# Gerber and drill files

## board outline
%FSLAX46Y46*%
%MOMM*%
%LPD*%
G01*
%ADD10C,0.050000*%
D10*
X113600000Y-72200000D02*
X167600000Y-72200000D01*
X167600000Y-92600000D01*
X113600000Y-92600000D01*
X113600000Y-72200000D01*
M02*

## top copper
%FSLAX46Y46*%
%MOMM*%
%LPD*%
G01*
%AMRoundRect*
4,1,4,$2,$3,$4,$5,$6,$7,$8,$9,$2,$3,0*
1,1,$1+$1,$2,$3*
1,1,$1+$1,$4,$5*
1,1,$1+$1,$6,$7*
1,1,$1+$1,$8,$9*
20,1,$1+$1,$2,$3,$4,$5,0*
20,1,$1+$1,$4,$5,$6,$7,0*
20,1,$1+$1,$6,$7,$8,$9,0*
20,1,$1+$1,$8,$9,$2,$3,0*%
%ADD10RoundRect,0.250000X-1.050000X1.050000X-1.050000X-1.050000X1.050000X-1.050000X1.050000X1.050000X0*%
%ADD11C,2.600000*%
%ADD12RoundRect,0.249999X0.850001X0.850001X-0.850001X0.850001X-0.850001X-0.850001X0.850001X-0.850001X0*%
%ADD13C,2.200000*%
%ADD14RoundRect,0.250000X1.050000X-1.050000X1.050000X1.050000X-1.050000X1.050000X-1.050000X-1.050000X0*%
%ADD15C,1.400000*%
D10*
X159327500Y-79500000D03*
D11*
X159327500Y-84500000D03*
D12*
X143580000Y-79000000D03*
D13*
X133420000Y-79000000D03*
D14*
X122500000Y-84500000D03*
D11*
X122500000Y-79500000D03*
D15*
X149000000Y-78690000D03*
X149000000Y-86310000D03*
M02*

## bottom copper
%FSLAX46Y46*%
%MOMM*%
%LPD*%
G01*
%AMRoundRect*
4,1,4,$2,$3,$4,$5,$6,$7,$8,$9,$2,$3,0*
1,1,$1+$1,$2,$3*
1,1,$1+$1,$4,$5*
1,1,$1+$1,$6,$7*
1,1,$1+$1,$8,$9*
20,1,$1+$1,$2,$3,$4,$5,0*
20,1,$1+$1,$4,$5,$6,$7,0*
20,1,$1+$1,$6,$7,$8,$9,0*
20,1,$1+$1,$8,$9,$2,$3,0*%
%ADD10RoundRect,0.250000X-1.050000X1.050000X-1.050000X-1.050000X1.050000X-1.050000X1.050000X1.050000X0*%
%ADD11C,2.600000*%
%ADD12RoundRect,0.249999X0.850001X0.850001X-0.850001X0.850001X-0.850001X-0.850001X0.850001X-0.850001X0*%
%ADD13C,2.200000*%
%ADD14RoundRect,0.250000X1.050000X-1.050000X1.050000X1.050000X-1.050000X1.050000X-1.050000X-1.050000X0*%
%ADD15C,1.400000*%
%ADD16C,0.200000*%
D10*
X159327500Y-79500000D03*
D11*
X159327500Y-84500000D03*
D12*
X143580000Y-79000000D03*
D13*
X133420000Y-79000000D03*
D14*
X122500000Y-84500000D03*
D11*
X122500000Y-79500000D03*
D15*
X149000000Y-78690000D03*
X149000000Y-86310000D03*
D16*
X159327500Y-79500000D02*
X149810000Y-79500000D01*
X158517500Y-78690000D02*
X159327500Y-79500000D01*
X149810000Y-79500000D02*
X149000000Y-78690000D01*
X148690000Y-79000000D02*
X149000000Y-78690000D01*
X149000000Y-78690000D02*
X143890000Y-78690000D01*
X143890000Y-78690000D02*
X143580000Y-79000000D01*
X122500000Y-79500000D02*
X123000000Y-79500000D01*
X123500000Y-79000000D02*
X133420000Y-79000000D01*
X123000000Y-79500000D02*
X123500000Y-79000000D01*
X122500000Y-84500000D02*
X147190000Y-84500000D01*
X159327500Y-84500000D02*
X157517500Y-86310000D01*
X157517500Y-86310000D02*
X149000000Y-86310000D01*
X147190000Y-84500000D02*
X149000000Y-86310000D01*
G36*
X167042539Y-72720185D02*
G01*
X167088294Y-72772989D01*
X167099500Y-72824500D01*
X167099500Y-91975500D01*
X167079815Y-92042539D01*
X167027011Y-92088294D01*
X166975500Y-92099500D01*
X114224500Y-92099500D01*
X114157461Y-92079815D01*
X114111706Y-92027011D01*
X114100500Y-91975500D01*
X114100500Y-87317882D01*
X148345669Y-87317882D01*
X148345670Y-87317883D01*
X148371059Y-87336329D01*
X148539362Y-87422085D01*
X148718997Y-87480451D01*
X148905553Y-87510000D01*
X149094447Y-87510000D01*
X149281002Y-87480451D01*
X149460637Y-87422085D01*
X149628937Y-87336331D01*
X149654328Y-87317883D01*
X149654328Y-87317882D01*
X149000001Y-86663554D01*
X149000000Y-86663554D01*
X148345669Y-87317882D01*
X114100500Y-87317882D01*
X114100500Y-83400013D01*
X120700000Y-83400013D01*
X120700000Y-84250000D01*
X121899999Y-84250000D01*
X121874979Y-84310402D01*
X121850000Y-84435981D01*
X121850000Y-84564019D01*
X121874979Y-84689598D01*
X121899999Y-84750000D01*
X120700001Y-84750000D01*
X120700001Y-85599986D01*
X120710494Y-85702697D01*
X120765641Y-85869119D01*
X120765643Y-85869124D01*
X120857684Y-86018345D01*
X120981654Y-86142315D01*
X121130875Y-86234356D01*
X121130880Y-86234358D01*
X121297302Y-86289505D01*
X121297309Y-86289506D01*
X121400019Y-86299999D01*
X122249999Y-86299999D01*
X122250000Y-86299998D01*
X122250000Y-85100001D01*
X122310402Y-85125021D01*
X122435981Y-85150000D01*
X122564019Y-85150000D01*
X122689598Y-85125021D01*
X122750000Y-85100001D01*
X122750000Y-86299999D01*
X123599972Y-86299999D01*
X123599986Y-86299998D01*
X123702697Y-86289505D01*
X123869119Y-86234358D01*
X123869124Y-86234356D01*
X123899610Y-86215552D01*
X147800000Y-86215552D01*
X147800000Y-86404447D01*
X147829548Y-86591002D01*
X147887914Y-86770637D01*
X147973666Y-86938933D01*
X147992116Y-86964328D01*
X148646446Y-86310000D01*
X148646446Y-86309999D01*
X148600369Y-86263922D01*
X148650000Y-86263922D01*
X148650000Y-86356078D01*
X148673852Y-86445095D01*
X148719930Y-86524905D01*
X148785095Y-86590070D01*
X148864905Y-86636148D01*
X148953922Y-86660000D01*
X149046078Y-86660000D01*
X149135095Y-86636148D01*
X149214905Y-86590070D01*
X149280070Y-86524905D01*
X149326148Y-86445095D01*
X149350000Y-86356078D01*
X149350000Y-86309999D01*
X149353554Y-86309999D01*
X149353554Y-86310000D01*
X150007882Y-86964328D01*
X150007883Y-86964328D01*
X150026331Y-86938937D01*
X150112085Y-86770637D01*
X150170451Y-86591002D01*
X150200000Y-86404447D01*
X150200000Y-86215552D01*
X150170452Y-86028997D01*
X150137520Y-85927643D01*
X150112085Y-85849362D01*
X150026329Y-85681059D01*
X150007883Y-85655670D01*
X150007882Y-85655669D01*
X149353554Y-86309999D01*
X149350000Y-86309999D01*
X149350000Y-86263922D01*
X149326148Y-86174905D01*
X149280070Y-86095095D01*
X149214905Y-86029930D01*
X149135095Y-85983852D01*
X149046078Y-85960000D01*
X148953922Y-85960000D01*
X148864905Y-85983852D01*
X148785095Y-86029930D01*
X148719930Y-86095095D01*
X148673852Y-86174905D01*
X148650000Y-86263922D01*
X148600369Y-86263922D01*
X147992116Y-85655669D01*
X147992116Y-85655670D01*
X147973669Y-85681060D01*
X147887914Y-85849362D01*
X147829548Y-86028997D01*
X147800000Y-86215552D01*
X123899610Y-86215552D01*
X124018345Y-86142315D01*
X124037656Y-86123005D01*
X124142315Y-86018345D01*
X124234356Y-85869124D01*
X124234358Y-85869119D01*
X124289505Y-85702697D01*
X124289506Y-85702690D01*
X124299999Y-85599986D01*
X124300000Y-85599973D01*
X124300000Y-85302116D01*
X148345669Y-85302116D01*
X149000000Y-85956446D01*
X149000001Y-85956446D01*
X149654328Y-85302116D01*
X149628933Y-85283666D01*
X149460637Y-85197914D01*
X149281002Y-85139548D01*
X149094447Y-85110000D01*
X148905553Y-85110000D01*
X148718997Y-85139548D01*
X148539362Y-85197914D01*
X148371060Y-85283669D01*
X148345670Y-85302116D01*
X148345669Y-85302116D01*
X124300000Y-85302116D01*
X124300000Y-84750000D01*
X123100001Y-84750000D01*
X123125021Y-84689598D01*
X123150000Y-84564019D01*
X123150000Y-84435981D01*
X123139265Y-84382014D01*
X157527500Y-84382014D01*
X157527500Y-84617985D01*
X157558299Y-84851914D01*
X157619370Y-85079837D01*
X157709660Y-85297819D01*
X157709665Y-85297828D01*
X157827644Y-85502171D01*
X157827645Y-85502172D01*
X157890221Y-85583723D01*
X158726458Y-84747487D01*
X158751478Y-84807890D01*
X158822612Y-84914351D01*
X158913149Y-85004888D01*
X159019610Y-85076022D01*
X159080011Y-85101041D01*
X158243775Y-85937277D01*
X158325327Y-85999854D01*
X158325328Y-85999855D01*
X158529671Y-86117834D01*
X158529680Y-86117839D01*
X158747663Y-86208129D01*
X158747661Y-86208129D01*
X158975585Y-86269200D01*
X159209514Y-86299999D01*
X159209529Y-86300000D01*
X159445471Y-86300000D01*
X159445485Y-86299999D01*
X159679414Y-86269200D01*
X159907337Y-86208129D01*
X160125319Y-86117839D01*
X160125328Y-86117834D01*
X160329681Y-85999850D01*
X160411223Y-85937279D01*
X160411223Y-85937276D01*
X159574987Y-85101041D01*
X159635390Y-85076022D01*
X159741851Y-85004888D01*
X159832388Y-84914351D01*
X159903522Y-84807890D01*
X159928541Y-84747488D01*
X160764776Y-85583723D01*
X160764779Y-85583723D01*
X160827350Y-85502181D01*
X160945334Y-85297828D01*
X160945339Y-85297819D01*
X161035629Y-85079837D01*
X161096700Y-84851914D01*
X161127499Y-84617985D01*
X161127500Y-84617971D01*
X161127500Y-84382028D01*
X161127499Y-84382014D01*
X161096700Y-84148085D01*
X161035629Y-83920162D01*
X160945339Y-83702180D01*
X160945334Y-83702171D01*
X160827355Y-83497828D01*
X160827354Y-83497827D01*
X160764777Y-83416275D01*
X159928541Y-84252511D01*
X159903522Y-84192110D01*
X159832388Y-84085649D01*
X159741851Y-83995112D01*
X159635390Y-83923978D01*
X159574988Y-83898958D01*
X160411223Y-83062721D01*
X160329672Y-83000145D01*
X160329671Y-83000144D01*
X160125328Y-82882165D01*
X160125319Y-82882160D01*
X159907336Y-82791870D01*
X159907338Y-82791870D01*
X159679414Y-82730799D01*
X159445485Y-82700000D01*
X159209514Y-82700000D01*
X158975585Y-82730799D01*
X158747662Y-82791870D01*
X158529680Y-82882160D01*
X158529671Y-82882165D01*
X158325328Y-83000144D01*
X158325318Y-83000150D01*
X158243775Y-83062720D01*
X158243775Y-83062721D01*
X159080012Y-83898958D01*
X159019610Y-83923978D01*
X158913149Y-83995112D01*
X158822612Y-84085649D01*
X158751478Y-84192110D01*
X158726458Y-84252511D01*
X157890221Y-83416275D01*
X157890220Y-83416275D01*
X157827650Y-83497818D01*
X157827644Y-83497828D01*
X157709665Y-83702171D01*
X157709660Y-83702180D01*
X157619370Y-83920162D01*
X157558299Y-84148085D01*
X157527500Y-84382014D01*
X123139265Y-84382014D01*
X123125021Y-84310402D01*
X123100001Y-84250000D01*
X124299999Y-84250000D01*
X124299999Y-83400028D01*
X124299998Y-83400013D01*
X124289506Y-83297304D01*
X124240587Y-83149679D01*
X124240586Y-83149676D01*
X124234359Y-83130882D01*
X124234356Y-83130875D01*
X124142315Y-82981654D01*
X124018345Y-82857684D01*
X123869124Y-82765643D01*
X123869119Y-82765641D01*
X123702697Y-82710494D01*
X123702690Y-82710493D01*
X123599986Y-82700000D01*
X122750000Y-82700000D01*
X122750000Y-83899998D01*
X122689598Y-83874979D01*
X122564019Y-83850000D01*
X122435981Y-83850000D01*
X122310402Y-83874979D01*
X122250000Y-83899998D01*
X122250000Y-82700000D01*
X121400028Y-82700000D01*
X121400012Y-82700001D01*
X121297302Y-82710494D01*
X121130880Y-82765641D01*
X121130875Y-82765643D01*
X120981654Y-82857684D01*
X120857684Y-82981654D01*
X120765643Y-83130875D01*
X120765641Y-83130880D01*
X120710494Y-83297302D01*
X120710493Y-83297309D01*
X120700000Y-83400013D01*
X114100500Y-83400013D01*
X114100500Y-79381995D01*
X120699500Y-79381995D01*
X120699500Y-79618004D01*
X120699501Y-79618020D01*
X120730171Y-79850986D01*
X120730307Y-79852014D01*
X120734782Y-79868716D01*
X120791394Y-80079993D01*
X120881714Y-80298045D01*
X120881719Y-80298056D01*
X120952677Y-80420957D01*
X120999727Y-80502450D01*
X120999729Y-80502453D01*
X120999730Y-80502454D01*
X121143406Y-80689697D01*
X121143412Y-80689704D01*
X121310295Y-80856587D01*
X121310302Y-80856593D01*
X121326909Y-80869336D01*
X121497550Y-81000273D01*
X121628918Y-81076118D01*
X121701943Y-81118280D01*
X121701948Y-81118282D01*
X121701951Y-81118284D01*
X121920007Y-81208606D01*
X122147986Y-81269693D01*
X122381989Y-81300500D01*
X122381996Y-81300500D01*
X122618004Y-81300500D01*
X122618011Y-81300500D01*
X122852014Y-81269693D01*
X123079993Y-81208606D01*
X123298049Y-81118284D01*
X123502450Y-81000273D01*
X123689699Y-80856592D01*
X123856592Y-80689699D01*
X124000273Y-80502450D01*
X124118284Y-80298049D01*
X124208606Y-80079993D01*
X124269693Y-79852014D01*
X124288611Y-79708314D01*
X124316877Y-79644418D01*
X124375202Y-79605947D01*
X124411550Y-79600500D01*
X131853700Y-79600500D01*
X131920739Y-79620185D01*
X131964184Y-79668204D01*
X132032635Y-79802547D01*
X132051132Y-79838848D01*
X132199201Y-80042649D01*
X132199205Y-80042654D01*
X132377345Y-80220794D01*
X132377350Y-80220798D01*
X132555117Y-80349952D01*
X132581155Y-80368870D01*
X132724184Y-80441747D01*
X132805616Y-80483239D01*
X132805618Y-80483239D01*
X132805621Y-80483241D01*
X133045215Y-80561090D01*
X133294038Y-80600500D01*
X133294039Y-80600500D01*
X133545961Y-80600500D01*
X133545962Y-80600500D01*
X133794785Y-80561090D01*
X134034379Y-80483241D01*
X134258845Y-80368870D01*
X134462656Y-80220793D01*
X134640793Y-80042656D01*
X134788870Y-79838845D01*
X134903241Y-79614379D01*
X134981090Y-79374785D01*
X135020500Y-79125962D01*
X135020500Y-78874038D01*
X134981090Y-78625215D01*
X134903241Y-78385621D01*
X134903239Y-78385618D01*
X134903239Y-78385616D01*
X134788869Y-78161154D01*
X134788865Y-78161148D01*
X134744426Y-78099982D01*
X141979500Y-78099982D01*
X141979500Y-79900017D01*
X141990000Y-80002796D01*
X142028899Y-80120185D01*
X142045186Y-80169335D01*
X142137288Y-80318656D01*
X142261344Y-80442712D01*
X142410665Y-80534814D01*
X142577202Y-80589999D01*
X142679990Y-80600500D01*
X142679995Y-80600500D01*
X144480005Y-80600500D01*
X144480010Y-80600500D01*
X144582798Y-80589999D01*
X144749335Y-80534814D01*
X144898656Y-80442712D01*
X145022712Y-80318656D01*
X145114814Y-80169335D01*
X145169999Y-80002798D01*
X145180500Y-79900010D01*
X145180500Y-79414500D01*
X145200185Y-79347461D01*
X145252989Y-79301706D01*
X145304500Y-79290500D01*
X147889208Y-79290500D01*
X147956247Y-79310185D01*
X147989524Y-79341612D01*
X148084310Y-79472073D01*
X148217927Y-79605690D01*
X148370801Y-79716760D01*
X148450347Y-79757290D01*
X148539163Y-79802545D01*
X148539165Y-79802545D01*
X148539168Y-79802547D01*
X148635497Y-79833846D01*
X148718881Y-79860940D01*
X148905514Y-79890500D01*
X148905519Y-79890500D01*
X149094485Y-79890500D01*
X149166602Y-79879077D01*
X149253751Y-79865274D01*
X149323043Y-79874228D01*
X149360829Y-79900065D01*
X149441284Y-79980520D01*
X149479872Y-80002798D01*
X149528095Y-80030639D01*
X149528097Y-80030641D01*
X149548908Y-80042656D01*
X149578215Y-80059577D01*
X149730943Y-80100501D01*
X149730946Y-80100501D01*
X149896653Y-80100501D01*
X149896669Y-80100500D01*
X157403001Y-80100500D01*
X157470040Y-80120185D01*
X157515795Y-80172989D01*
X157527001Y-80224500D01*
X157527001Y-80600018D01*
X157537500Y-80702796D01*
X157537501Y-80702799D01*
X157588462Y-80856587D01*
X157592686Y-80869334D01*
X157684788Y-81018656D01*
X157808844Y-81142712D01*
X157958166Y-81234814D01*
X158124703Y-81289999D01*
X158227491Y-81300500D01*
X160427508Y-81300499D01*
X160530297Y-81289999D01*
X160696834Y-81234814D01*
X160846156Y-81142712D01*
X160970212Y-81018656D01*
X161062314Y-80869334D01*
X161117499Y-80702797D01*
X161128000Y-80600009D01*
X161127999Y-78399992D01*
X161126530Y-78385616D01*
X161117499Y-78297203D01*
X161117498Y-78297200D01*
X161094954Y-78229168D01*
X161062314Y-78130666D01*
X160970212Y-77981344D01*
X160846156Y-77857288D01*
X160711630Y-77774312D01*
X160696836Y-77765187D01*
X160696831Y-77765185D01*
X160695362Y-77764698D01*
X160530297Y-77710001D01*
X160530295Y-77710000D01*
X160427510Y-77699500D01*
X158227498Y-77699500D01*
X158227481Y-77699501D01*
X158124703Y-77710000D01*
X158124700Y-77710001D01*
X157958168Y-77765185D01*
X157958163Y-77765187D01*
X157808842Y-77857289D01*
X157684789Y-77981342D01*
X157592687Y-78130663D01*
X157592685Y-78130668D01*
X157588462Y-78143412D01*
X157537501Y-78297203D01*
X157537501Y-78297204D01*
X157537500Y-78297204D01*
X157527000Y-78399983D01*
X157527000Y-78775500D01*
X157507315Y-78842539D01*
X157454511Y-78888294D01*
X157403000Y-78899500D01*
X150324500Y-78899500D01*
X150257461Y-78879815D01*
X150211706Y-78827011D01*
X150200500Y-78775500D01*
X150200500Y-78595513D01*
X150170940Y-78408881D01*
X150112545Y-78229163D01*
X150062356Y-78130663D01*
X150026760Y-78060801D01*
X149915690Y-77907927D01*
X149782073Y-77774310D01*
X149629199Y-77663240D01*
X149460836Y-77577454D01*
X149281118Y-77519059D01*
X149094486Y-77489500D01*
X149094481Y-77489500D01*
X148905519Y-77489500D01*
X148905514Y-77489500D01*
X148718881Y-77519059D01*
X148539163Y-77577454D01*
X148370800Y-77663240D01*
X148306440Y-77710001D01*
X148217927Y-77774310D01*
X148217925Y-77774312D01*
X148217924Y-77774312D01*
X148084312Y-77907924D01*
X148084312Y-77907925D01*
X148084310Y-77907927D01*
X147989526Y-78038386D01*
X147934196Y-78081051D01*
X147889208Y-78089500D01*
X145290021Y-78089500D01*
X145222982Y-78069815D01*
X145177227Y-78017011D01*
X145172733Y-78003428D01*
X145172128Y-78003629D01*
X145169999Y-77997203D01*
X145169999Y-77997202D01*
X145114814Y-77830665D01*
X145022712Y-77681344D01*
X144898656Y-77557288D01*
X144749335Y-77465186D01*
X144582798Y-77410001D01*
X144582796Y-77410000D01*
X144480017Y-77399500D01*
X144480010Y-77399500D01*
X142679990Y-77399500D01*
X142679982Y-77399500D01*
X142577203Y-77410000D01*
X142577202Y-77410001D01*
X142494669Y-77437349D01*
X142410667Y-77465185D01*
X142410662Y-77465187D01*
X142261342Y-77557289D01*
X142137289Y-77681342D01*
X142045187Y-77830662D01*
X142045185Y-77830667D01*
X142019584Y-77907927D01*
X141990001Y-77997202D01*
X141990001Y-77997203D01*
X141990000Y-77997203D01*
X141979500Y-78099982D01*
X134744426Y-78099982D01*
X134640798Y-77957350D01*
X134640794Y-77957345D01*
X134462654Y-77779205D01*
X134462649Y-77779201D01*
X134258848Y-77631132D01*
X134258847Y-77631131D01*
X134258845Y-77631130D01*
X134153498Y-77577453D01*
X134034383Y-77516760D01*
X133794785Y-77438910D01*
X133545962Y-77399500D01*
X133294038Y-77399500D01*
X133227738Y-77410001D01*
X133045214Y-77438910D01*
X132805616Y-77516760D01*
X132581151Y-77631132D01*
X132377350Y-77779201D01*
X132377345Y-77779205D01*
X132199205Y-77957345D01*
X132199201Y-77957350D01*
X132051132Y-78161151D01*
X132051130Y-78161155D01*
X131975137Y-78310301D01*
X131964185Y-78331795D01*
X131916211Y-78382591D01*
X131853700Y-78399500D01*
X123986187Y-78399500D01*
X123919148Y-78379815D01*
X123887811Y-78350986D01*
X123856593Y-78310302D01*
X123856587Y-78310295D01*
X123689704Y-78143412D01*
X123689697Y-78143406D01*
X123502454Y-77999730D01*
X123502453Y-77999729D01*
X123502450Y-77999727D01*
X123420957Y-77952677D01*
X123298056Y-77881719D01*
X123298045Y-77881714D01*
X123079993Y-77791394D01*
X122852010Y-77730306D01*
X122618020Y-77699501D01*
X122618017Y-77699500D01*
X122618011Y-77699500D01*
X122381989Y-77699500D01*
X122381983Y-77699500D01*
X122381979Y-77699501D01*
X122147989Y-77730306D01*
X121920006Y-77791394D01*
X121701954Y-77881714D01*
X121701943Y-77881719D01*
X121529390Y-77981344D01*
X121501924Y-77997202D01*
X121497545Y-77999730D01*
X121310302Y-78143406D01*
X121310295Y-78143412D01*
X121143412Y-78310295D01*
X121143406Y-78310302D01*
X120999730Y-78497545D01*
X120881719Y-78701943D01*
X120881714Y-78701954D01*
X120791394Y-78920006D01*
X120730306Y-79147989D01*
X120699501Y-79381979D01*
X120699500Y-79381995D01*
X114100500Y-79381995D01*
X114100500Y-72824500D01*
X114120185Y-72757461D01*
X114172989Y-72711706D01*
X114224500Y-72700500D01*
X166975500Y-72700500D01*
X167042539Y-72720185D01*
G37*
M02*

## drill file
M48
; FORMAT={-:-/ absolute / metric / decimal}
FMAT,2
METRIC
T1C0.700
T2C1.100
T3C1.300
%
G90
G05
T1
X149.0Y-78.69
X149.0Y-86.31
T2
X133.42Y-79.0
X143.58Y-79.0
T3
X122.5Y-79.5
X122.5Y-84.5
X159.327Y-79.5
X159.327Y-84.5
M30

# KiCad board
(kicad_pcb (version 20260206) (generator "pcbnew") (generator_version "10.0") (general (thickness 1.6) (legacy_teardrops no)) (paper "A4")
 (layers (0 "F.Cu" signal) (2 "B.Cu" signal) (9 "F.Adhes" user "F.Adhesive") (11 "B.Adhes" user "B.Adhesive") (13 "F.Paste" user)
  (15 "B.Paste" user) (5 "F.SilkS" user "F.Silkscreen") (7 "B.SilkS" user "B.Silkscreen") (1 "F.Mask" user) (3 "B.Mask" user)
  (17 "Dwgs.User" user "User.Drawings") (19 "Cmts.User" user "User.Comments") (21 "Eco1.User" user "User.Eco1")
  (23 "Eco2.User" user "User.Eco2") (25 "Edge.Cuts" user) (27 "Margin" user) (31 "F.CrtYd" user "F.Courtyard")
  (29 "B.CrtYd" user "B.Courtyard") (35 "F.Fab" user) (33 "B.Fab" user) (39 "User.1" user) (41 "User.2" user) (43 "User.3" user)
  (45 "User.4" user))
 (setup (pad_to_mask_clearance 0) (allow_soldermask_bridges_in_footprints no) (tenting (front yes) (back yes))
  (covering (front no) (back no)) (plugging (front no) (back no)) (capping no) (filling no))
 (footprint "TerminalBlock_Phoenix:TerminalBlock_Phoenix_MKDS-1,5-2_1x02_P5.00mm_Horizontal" (layer "F.Cu") (at 159.3275 79.5 -90)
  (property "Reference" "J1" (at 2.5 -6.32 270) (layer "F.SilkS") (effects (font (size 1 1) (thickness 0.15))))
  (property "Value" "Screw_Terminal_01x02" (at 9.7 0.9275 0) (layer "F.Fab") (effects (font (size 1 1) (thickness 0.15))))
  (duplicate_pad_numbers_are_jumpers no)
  (pad "1" thru_hole roundrect (at 0 0 270) (size 2.6 2.6) (drill 1.3) (layers "*.Cu" "*.Mask") (remove_unused_layers no)
   (roundrect_rratio 0.096154) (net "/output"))
  (pad "2" thru_hole circle (at 5 0 270) (size 2.6 2.6) (drill 1.3) (layers "*.Cu" "*.Mask") (remove_unused_layers no) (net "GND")))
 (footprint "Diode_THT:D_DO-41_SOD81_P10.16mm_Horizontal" (layer "F.Cu") (at 143.58 79 180)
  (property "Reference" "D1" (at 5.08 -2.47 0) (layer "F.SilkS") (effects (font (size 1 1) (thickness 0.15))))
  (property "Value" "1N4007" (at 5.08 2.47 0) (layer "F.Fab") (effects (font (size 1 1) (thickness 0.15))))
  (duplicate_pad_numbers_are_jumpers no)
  (pad "1" thru_hole roundrect (at 0 0 180) (size 2.2 2.2) (drill 1.1) (layers "*.Cu" "*.Mask") (remove_unused_layers no)
   (roundrect_rratio 0.113636) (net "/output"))
  (pad "2" thru_hole circle (at 10.16 0 180) (size 2.2 2.2) (drill 1.1) (layers "*.Cu" "*.Mask") (remove_unused_layers no) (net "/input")))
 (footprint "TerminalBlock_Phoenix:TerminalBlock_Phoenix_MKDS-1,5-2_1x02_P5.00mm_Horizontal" (layer "F.Cu") (at 122.5 84.5 90)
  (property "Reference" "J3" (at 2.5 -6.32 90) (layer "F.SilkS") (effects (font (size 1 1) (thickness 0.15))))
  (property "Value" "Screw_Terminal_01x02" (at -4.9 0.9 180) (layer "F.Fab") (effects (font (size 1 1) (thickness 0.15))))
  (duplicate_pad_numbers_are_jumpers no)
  (pad "1" thru_hole roundrect (at 0 0 90) (size 2.6 2.6) (drill 1.3) (layers "*.Cu" "*.Mask") (remove_unused_layers no)
   (roundrect_rratio 0.096154) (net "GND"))
  (pad "2" thru_hole circle (at 5 0 90) (size 2.6 2.6) (drill 1.3) (layers "*.Cu" "*.Mask") (remove_unused_layers no) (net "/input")))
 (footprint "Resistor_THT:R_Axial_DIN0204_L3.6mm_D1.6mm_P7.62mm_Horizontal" (layer "F.Cu") (at 149 78.69 -90)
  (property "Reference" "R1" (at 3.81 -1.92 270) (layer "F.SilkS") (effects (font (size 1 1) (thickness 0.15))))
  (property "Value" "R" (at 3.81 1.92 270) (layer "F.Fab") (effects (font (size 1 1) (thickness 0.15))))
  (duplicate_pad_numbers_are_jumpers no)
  (pad "1" thru_hole circle (at 0 0 270) (size 1.4 1.4) (drill 0.7) (layers "*.Cu" "*.Mask") (remove_unused_layers no) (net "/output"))
  (pad "2" thru_hole circle (at 7.62 0 270) (size 1.4 1.4) (drill 0.7) (layers "*.Cu" "*.Mask") (remove_unused_layers no) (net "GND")))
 (gr_rect (start 113.6 72.2) (end 167.6 92.6) (stroke (width 0.05) (type default)) (fill no) (layer "Edge.Cuts"))
 (segment (start 159.3275 79.5) (end 149.81 79.5) (width 0.2) (layer "B.Cu") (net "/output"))
 (segment (start 158.5175 78.69) (end 159.3275 79.5) (width 0.2) (layer "B.Cu") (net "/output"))
 (segment (start 149.81 79.5) (end 149 78.69) (width 0.2) (layer "B.Cu") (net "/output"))
 (segment (start 148.69 79) (end 149 78.69) (width 0.2) (layer "B.Cu") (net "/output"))
 (segment (start 149 78.69) (end 143.89 78.69) (width 0.2) (layer "B.Cu") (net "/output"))
 (segment (start 143.89 78.69) (end 143.58 79) (width 0.2) (layer "B.Cu") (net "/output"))
 (segment (start 122.5 79.5) (end 123 79.5) (width 0.2) (layer "B.Cu") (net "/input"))
 (segment (start 123.5 79) (end 133.42 79) (width 0.2) (layer "B.Cu") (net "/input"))
 (segment (start 123 79.5) (end 123.5 79) (width 0.2) (layer "B.Cu") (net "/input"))
 (segment (start 122.5 84.5) (end 147.19 84.5) (width 0.2) (layer "B.Cu") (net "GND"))
 (segment (start 159.3275 84.5) (end 157.5175 86.31) (width 0.2) (layer "B.Cu") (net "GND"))
 (segment (start 157.5175 86.31) (end 149 86.31) (width 0.2) (layer "B.Cu") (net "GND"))
 (segment (start 147.19 84.5) (end 149 86.31) (width 0.2) (layer "B.Cu") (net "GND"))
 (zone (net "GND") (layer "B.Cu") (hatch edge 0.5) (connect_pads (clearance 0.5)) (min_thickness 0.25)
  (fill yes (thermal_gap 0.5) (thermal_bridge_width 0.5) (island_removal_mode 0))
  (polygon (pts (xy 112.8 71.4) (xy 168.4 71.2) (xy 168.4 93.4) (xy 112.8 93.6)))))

